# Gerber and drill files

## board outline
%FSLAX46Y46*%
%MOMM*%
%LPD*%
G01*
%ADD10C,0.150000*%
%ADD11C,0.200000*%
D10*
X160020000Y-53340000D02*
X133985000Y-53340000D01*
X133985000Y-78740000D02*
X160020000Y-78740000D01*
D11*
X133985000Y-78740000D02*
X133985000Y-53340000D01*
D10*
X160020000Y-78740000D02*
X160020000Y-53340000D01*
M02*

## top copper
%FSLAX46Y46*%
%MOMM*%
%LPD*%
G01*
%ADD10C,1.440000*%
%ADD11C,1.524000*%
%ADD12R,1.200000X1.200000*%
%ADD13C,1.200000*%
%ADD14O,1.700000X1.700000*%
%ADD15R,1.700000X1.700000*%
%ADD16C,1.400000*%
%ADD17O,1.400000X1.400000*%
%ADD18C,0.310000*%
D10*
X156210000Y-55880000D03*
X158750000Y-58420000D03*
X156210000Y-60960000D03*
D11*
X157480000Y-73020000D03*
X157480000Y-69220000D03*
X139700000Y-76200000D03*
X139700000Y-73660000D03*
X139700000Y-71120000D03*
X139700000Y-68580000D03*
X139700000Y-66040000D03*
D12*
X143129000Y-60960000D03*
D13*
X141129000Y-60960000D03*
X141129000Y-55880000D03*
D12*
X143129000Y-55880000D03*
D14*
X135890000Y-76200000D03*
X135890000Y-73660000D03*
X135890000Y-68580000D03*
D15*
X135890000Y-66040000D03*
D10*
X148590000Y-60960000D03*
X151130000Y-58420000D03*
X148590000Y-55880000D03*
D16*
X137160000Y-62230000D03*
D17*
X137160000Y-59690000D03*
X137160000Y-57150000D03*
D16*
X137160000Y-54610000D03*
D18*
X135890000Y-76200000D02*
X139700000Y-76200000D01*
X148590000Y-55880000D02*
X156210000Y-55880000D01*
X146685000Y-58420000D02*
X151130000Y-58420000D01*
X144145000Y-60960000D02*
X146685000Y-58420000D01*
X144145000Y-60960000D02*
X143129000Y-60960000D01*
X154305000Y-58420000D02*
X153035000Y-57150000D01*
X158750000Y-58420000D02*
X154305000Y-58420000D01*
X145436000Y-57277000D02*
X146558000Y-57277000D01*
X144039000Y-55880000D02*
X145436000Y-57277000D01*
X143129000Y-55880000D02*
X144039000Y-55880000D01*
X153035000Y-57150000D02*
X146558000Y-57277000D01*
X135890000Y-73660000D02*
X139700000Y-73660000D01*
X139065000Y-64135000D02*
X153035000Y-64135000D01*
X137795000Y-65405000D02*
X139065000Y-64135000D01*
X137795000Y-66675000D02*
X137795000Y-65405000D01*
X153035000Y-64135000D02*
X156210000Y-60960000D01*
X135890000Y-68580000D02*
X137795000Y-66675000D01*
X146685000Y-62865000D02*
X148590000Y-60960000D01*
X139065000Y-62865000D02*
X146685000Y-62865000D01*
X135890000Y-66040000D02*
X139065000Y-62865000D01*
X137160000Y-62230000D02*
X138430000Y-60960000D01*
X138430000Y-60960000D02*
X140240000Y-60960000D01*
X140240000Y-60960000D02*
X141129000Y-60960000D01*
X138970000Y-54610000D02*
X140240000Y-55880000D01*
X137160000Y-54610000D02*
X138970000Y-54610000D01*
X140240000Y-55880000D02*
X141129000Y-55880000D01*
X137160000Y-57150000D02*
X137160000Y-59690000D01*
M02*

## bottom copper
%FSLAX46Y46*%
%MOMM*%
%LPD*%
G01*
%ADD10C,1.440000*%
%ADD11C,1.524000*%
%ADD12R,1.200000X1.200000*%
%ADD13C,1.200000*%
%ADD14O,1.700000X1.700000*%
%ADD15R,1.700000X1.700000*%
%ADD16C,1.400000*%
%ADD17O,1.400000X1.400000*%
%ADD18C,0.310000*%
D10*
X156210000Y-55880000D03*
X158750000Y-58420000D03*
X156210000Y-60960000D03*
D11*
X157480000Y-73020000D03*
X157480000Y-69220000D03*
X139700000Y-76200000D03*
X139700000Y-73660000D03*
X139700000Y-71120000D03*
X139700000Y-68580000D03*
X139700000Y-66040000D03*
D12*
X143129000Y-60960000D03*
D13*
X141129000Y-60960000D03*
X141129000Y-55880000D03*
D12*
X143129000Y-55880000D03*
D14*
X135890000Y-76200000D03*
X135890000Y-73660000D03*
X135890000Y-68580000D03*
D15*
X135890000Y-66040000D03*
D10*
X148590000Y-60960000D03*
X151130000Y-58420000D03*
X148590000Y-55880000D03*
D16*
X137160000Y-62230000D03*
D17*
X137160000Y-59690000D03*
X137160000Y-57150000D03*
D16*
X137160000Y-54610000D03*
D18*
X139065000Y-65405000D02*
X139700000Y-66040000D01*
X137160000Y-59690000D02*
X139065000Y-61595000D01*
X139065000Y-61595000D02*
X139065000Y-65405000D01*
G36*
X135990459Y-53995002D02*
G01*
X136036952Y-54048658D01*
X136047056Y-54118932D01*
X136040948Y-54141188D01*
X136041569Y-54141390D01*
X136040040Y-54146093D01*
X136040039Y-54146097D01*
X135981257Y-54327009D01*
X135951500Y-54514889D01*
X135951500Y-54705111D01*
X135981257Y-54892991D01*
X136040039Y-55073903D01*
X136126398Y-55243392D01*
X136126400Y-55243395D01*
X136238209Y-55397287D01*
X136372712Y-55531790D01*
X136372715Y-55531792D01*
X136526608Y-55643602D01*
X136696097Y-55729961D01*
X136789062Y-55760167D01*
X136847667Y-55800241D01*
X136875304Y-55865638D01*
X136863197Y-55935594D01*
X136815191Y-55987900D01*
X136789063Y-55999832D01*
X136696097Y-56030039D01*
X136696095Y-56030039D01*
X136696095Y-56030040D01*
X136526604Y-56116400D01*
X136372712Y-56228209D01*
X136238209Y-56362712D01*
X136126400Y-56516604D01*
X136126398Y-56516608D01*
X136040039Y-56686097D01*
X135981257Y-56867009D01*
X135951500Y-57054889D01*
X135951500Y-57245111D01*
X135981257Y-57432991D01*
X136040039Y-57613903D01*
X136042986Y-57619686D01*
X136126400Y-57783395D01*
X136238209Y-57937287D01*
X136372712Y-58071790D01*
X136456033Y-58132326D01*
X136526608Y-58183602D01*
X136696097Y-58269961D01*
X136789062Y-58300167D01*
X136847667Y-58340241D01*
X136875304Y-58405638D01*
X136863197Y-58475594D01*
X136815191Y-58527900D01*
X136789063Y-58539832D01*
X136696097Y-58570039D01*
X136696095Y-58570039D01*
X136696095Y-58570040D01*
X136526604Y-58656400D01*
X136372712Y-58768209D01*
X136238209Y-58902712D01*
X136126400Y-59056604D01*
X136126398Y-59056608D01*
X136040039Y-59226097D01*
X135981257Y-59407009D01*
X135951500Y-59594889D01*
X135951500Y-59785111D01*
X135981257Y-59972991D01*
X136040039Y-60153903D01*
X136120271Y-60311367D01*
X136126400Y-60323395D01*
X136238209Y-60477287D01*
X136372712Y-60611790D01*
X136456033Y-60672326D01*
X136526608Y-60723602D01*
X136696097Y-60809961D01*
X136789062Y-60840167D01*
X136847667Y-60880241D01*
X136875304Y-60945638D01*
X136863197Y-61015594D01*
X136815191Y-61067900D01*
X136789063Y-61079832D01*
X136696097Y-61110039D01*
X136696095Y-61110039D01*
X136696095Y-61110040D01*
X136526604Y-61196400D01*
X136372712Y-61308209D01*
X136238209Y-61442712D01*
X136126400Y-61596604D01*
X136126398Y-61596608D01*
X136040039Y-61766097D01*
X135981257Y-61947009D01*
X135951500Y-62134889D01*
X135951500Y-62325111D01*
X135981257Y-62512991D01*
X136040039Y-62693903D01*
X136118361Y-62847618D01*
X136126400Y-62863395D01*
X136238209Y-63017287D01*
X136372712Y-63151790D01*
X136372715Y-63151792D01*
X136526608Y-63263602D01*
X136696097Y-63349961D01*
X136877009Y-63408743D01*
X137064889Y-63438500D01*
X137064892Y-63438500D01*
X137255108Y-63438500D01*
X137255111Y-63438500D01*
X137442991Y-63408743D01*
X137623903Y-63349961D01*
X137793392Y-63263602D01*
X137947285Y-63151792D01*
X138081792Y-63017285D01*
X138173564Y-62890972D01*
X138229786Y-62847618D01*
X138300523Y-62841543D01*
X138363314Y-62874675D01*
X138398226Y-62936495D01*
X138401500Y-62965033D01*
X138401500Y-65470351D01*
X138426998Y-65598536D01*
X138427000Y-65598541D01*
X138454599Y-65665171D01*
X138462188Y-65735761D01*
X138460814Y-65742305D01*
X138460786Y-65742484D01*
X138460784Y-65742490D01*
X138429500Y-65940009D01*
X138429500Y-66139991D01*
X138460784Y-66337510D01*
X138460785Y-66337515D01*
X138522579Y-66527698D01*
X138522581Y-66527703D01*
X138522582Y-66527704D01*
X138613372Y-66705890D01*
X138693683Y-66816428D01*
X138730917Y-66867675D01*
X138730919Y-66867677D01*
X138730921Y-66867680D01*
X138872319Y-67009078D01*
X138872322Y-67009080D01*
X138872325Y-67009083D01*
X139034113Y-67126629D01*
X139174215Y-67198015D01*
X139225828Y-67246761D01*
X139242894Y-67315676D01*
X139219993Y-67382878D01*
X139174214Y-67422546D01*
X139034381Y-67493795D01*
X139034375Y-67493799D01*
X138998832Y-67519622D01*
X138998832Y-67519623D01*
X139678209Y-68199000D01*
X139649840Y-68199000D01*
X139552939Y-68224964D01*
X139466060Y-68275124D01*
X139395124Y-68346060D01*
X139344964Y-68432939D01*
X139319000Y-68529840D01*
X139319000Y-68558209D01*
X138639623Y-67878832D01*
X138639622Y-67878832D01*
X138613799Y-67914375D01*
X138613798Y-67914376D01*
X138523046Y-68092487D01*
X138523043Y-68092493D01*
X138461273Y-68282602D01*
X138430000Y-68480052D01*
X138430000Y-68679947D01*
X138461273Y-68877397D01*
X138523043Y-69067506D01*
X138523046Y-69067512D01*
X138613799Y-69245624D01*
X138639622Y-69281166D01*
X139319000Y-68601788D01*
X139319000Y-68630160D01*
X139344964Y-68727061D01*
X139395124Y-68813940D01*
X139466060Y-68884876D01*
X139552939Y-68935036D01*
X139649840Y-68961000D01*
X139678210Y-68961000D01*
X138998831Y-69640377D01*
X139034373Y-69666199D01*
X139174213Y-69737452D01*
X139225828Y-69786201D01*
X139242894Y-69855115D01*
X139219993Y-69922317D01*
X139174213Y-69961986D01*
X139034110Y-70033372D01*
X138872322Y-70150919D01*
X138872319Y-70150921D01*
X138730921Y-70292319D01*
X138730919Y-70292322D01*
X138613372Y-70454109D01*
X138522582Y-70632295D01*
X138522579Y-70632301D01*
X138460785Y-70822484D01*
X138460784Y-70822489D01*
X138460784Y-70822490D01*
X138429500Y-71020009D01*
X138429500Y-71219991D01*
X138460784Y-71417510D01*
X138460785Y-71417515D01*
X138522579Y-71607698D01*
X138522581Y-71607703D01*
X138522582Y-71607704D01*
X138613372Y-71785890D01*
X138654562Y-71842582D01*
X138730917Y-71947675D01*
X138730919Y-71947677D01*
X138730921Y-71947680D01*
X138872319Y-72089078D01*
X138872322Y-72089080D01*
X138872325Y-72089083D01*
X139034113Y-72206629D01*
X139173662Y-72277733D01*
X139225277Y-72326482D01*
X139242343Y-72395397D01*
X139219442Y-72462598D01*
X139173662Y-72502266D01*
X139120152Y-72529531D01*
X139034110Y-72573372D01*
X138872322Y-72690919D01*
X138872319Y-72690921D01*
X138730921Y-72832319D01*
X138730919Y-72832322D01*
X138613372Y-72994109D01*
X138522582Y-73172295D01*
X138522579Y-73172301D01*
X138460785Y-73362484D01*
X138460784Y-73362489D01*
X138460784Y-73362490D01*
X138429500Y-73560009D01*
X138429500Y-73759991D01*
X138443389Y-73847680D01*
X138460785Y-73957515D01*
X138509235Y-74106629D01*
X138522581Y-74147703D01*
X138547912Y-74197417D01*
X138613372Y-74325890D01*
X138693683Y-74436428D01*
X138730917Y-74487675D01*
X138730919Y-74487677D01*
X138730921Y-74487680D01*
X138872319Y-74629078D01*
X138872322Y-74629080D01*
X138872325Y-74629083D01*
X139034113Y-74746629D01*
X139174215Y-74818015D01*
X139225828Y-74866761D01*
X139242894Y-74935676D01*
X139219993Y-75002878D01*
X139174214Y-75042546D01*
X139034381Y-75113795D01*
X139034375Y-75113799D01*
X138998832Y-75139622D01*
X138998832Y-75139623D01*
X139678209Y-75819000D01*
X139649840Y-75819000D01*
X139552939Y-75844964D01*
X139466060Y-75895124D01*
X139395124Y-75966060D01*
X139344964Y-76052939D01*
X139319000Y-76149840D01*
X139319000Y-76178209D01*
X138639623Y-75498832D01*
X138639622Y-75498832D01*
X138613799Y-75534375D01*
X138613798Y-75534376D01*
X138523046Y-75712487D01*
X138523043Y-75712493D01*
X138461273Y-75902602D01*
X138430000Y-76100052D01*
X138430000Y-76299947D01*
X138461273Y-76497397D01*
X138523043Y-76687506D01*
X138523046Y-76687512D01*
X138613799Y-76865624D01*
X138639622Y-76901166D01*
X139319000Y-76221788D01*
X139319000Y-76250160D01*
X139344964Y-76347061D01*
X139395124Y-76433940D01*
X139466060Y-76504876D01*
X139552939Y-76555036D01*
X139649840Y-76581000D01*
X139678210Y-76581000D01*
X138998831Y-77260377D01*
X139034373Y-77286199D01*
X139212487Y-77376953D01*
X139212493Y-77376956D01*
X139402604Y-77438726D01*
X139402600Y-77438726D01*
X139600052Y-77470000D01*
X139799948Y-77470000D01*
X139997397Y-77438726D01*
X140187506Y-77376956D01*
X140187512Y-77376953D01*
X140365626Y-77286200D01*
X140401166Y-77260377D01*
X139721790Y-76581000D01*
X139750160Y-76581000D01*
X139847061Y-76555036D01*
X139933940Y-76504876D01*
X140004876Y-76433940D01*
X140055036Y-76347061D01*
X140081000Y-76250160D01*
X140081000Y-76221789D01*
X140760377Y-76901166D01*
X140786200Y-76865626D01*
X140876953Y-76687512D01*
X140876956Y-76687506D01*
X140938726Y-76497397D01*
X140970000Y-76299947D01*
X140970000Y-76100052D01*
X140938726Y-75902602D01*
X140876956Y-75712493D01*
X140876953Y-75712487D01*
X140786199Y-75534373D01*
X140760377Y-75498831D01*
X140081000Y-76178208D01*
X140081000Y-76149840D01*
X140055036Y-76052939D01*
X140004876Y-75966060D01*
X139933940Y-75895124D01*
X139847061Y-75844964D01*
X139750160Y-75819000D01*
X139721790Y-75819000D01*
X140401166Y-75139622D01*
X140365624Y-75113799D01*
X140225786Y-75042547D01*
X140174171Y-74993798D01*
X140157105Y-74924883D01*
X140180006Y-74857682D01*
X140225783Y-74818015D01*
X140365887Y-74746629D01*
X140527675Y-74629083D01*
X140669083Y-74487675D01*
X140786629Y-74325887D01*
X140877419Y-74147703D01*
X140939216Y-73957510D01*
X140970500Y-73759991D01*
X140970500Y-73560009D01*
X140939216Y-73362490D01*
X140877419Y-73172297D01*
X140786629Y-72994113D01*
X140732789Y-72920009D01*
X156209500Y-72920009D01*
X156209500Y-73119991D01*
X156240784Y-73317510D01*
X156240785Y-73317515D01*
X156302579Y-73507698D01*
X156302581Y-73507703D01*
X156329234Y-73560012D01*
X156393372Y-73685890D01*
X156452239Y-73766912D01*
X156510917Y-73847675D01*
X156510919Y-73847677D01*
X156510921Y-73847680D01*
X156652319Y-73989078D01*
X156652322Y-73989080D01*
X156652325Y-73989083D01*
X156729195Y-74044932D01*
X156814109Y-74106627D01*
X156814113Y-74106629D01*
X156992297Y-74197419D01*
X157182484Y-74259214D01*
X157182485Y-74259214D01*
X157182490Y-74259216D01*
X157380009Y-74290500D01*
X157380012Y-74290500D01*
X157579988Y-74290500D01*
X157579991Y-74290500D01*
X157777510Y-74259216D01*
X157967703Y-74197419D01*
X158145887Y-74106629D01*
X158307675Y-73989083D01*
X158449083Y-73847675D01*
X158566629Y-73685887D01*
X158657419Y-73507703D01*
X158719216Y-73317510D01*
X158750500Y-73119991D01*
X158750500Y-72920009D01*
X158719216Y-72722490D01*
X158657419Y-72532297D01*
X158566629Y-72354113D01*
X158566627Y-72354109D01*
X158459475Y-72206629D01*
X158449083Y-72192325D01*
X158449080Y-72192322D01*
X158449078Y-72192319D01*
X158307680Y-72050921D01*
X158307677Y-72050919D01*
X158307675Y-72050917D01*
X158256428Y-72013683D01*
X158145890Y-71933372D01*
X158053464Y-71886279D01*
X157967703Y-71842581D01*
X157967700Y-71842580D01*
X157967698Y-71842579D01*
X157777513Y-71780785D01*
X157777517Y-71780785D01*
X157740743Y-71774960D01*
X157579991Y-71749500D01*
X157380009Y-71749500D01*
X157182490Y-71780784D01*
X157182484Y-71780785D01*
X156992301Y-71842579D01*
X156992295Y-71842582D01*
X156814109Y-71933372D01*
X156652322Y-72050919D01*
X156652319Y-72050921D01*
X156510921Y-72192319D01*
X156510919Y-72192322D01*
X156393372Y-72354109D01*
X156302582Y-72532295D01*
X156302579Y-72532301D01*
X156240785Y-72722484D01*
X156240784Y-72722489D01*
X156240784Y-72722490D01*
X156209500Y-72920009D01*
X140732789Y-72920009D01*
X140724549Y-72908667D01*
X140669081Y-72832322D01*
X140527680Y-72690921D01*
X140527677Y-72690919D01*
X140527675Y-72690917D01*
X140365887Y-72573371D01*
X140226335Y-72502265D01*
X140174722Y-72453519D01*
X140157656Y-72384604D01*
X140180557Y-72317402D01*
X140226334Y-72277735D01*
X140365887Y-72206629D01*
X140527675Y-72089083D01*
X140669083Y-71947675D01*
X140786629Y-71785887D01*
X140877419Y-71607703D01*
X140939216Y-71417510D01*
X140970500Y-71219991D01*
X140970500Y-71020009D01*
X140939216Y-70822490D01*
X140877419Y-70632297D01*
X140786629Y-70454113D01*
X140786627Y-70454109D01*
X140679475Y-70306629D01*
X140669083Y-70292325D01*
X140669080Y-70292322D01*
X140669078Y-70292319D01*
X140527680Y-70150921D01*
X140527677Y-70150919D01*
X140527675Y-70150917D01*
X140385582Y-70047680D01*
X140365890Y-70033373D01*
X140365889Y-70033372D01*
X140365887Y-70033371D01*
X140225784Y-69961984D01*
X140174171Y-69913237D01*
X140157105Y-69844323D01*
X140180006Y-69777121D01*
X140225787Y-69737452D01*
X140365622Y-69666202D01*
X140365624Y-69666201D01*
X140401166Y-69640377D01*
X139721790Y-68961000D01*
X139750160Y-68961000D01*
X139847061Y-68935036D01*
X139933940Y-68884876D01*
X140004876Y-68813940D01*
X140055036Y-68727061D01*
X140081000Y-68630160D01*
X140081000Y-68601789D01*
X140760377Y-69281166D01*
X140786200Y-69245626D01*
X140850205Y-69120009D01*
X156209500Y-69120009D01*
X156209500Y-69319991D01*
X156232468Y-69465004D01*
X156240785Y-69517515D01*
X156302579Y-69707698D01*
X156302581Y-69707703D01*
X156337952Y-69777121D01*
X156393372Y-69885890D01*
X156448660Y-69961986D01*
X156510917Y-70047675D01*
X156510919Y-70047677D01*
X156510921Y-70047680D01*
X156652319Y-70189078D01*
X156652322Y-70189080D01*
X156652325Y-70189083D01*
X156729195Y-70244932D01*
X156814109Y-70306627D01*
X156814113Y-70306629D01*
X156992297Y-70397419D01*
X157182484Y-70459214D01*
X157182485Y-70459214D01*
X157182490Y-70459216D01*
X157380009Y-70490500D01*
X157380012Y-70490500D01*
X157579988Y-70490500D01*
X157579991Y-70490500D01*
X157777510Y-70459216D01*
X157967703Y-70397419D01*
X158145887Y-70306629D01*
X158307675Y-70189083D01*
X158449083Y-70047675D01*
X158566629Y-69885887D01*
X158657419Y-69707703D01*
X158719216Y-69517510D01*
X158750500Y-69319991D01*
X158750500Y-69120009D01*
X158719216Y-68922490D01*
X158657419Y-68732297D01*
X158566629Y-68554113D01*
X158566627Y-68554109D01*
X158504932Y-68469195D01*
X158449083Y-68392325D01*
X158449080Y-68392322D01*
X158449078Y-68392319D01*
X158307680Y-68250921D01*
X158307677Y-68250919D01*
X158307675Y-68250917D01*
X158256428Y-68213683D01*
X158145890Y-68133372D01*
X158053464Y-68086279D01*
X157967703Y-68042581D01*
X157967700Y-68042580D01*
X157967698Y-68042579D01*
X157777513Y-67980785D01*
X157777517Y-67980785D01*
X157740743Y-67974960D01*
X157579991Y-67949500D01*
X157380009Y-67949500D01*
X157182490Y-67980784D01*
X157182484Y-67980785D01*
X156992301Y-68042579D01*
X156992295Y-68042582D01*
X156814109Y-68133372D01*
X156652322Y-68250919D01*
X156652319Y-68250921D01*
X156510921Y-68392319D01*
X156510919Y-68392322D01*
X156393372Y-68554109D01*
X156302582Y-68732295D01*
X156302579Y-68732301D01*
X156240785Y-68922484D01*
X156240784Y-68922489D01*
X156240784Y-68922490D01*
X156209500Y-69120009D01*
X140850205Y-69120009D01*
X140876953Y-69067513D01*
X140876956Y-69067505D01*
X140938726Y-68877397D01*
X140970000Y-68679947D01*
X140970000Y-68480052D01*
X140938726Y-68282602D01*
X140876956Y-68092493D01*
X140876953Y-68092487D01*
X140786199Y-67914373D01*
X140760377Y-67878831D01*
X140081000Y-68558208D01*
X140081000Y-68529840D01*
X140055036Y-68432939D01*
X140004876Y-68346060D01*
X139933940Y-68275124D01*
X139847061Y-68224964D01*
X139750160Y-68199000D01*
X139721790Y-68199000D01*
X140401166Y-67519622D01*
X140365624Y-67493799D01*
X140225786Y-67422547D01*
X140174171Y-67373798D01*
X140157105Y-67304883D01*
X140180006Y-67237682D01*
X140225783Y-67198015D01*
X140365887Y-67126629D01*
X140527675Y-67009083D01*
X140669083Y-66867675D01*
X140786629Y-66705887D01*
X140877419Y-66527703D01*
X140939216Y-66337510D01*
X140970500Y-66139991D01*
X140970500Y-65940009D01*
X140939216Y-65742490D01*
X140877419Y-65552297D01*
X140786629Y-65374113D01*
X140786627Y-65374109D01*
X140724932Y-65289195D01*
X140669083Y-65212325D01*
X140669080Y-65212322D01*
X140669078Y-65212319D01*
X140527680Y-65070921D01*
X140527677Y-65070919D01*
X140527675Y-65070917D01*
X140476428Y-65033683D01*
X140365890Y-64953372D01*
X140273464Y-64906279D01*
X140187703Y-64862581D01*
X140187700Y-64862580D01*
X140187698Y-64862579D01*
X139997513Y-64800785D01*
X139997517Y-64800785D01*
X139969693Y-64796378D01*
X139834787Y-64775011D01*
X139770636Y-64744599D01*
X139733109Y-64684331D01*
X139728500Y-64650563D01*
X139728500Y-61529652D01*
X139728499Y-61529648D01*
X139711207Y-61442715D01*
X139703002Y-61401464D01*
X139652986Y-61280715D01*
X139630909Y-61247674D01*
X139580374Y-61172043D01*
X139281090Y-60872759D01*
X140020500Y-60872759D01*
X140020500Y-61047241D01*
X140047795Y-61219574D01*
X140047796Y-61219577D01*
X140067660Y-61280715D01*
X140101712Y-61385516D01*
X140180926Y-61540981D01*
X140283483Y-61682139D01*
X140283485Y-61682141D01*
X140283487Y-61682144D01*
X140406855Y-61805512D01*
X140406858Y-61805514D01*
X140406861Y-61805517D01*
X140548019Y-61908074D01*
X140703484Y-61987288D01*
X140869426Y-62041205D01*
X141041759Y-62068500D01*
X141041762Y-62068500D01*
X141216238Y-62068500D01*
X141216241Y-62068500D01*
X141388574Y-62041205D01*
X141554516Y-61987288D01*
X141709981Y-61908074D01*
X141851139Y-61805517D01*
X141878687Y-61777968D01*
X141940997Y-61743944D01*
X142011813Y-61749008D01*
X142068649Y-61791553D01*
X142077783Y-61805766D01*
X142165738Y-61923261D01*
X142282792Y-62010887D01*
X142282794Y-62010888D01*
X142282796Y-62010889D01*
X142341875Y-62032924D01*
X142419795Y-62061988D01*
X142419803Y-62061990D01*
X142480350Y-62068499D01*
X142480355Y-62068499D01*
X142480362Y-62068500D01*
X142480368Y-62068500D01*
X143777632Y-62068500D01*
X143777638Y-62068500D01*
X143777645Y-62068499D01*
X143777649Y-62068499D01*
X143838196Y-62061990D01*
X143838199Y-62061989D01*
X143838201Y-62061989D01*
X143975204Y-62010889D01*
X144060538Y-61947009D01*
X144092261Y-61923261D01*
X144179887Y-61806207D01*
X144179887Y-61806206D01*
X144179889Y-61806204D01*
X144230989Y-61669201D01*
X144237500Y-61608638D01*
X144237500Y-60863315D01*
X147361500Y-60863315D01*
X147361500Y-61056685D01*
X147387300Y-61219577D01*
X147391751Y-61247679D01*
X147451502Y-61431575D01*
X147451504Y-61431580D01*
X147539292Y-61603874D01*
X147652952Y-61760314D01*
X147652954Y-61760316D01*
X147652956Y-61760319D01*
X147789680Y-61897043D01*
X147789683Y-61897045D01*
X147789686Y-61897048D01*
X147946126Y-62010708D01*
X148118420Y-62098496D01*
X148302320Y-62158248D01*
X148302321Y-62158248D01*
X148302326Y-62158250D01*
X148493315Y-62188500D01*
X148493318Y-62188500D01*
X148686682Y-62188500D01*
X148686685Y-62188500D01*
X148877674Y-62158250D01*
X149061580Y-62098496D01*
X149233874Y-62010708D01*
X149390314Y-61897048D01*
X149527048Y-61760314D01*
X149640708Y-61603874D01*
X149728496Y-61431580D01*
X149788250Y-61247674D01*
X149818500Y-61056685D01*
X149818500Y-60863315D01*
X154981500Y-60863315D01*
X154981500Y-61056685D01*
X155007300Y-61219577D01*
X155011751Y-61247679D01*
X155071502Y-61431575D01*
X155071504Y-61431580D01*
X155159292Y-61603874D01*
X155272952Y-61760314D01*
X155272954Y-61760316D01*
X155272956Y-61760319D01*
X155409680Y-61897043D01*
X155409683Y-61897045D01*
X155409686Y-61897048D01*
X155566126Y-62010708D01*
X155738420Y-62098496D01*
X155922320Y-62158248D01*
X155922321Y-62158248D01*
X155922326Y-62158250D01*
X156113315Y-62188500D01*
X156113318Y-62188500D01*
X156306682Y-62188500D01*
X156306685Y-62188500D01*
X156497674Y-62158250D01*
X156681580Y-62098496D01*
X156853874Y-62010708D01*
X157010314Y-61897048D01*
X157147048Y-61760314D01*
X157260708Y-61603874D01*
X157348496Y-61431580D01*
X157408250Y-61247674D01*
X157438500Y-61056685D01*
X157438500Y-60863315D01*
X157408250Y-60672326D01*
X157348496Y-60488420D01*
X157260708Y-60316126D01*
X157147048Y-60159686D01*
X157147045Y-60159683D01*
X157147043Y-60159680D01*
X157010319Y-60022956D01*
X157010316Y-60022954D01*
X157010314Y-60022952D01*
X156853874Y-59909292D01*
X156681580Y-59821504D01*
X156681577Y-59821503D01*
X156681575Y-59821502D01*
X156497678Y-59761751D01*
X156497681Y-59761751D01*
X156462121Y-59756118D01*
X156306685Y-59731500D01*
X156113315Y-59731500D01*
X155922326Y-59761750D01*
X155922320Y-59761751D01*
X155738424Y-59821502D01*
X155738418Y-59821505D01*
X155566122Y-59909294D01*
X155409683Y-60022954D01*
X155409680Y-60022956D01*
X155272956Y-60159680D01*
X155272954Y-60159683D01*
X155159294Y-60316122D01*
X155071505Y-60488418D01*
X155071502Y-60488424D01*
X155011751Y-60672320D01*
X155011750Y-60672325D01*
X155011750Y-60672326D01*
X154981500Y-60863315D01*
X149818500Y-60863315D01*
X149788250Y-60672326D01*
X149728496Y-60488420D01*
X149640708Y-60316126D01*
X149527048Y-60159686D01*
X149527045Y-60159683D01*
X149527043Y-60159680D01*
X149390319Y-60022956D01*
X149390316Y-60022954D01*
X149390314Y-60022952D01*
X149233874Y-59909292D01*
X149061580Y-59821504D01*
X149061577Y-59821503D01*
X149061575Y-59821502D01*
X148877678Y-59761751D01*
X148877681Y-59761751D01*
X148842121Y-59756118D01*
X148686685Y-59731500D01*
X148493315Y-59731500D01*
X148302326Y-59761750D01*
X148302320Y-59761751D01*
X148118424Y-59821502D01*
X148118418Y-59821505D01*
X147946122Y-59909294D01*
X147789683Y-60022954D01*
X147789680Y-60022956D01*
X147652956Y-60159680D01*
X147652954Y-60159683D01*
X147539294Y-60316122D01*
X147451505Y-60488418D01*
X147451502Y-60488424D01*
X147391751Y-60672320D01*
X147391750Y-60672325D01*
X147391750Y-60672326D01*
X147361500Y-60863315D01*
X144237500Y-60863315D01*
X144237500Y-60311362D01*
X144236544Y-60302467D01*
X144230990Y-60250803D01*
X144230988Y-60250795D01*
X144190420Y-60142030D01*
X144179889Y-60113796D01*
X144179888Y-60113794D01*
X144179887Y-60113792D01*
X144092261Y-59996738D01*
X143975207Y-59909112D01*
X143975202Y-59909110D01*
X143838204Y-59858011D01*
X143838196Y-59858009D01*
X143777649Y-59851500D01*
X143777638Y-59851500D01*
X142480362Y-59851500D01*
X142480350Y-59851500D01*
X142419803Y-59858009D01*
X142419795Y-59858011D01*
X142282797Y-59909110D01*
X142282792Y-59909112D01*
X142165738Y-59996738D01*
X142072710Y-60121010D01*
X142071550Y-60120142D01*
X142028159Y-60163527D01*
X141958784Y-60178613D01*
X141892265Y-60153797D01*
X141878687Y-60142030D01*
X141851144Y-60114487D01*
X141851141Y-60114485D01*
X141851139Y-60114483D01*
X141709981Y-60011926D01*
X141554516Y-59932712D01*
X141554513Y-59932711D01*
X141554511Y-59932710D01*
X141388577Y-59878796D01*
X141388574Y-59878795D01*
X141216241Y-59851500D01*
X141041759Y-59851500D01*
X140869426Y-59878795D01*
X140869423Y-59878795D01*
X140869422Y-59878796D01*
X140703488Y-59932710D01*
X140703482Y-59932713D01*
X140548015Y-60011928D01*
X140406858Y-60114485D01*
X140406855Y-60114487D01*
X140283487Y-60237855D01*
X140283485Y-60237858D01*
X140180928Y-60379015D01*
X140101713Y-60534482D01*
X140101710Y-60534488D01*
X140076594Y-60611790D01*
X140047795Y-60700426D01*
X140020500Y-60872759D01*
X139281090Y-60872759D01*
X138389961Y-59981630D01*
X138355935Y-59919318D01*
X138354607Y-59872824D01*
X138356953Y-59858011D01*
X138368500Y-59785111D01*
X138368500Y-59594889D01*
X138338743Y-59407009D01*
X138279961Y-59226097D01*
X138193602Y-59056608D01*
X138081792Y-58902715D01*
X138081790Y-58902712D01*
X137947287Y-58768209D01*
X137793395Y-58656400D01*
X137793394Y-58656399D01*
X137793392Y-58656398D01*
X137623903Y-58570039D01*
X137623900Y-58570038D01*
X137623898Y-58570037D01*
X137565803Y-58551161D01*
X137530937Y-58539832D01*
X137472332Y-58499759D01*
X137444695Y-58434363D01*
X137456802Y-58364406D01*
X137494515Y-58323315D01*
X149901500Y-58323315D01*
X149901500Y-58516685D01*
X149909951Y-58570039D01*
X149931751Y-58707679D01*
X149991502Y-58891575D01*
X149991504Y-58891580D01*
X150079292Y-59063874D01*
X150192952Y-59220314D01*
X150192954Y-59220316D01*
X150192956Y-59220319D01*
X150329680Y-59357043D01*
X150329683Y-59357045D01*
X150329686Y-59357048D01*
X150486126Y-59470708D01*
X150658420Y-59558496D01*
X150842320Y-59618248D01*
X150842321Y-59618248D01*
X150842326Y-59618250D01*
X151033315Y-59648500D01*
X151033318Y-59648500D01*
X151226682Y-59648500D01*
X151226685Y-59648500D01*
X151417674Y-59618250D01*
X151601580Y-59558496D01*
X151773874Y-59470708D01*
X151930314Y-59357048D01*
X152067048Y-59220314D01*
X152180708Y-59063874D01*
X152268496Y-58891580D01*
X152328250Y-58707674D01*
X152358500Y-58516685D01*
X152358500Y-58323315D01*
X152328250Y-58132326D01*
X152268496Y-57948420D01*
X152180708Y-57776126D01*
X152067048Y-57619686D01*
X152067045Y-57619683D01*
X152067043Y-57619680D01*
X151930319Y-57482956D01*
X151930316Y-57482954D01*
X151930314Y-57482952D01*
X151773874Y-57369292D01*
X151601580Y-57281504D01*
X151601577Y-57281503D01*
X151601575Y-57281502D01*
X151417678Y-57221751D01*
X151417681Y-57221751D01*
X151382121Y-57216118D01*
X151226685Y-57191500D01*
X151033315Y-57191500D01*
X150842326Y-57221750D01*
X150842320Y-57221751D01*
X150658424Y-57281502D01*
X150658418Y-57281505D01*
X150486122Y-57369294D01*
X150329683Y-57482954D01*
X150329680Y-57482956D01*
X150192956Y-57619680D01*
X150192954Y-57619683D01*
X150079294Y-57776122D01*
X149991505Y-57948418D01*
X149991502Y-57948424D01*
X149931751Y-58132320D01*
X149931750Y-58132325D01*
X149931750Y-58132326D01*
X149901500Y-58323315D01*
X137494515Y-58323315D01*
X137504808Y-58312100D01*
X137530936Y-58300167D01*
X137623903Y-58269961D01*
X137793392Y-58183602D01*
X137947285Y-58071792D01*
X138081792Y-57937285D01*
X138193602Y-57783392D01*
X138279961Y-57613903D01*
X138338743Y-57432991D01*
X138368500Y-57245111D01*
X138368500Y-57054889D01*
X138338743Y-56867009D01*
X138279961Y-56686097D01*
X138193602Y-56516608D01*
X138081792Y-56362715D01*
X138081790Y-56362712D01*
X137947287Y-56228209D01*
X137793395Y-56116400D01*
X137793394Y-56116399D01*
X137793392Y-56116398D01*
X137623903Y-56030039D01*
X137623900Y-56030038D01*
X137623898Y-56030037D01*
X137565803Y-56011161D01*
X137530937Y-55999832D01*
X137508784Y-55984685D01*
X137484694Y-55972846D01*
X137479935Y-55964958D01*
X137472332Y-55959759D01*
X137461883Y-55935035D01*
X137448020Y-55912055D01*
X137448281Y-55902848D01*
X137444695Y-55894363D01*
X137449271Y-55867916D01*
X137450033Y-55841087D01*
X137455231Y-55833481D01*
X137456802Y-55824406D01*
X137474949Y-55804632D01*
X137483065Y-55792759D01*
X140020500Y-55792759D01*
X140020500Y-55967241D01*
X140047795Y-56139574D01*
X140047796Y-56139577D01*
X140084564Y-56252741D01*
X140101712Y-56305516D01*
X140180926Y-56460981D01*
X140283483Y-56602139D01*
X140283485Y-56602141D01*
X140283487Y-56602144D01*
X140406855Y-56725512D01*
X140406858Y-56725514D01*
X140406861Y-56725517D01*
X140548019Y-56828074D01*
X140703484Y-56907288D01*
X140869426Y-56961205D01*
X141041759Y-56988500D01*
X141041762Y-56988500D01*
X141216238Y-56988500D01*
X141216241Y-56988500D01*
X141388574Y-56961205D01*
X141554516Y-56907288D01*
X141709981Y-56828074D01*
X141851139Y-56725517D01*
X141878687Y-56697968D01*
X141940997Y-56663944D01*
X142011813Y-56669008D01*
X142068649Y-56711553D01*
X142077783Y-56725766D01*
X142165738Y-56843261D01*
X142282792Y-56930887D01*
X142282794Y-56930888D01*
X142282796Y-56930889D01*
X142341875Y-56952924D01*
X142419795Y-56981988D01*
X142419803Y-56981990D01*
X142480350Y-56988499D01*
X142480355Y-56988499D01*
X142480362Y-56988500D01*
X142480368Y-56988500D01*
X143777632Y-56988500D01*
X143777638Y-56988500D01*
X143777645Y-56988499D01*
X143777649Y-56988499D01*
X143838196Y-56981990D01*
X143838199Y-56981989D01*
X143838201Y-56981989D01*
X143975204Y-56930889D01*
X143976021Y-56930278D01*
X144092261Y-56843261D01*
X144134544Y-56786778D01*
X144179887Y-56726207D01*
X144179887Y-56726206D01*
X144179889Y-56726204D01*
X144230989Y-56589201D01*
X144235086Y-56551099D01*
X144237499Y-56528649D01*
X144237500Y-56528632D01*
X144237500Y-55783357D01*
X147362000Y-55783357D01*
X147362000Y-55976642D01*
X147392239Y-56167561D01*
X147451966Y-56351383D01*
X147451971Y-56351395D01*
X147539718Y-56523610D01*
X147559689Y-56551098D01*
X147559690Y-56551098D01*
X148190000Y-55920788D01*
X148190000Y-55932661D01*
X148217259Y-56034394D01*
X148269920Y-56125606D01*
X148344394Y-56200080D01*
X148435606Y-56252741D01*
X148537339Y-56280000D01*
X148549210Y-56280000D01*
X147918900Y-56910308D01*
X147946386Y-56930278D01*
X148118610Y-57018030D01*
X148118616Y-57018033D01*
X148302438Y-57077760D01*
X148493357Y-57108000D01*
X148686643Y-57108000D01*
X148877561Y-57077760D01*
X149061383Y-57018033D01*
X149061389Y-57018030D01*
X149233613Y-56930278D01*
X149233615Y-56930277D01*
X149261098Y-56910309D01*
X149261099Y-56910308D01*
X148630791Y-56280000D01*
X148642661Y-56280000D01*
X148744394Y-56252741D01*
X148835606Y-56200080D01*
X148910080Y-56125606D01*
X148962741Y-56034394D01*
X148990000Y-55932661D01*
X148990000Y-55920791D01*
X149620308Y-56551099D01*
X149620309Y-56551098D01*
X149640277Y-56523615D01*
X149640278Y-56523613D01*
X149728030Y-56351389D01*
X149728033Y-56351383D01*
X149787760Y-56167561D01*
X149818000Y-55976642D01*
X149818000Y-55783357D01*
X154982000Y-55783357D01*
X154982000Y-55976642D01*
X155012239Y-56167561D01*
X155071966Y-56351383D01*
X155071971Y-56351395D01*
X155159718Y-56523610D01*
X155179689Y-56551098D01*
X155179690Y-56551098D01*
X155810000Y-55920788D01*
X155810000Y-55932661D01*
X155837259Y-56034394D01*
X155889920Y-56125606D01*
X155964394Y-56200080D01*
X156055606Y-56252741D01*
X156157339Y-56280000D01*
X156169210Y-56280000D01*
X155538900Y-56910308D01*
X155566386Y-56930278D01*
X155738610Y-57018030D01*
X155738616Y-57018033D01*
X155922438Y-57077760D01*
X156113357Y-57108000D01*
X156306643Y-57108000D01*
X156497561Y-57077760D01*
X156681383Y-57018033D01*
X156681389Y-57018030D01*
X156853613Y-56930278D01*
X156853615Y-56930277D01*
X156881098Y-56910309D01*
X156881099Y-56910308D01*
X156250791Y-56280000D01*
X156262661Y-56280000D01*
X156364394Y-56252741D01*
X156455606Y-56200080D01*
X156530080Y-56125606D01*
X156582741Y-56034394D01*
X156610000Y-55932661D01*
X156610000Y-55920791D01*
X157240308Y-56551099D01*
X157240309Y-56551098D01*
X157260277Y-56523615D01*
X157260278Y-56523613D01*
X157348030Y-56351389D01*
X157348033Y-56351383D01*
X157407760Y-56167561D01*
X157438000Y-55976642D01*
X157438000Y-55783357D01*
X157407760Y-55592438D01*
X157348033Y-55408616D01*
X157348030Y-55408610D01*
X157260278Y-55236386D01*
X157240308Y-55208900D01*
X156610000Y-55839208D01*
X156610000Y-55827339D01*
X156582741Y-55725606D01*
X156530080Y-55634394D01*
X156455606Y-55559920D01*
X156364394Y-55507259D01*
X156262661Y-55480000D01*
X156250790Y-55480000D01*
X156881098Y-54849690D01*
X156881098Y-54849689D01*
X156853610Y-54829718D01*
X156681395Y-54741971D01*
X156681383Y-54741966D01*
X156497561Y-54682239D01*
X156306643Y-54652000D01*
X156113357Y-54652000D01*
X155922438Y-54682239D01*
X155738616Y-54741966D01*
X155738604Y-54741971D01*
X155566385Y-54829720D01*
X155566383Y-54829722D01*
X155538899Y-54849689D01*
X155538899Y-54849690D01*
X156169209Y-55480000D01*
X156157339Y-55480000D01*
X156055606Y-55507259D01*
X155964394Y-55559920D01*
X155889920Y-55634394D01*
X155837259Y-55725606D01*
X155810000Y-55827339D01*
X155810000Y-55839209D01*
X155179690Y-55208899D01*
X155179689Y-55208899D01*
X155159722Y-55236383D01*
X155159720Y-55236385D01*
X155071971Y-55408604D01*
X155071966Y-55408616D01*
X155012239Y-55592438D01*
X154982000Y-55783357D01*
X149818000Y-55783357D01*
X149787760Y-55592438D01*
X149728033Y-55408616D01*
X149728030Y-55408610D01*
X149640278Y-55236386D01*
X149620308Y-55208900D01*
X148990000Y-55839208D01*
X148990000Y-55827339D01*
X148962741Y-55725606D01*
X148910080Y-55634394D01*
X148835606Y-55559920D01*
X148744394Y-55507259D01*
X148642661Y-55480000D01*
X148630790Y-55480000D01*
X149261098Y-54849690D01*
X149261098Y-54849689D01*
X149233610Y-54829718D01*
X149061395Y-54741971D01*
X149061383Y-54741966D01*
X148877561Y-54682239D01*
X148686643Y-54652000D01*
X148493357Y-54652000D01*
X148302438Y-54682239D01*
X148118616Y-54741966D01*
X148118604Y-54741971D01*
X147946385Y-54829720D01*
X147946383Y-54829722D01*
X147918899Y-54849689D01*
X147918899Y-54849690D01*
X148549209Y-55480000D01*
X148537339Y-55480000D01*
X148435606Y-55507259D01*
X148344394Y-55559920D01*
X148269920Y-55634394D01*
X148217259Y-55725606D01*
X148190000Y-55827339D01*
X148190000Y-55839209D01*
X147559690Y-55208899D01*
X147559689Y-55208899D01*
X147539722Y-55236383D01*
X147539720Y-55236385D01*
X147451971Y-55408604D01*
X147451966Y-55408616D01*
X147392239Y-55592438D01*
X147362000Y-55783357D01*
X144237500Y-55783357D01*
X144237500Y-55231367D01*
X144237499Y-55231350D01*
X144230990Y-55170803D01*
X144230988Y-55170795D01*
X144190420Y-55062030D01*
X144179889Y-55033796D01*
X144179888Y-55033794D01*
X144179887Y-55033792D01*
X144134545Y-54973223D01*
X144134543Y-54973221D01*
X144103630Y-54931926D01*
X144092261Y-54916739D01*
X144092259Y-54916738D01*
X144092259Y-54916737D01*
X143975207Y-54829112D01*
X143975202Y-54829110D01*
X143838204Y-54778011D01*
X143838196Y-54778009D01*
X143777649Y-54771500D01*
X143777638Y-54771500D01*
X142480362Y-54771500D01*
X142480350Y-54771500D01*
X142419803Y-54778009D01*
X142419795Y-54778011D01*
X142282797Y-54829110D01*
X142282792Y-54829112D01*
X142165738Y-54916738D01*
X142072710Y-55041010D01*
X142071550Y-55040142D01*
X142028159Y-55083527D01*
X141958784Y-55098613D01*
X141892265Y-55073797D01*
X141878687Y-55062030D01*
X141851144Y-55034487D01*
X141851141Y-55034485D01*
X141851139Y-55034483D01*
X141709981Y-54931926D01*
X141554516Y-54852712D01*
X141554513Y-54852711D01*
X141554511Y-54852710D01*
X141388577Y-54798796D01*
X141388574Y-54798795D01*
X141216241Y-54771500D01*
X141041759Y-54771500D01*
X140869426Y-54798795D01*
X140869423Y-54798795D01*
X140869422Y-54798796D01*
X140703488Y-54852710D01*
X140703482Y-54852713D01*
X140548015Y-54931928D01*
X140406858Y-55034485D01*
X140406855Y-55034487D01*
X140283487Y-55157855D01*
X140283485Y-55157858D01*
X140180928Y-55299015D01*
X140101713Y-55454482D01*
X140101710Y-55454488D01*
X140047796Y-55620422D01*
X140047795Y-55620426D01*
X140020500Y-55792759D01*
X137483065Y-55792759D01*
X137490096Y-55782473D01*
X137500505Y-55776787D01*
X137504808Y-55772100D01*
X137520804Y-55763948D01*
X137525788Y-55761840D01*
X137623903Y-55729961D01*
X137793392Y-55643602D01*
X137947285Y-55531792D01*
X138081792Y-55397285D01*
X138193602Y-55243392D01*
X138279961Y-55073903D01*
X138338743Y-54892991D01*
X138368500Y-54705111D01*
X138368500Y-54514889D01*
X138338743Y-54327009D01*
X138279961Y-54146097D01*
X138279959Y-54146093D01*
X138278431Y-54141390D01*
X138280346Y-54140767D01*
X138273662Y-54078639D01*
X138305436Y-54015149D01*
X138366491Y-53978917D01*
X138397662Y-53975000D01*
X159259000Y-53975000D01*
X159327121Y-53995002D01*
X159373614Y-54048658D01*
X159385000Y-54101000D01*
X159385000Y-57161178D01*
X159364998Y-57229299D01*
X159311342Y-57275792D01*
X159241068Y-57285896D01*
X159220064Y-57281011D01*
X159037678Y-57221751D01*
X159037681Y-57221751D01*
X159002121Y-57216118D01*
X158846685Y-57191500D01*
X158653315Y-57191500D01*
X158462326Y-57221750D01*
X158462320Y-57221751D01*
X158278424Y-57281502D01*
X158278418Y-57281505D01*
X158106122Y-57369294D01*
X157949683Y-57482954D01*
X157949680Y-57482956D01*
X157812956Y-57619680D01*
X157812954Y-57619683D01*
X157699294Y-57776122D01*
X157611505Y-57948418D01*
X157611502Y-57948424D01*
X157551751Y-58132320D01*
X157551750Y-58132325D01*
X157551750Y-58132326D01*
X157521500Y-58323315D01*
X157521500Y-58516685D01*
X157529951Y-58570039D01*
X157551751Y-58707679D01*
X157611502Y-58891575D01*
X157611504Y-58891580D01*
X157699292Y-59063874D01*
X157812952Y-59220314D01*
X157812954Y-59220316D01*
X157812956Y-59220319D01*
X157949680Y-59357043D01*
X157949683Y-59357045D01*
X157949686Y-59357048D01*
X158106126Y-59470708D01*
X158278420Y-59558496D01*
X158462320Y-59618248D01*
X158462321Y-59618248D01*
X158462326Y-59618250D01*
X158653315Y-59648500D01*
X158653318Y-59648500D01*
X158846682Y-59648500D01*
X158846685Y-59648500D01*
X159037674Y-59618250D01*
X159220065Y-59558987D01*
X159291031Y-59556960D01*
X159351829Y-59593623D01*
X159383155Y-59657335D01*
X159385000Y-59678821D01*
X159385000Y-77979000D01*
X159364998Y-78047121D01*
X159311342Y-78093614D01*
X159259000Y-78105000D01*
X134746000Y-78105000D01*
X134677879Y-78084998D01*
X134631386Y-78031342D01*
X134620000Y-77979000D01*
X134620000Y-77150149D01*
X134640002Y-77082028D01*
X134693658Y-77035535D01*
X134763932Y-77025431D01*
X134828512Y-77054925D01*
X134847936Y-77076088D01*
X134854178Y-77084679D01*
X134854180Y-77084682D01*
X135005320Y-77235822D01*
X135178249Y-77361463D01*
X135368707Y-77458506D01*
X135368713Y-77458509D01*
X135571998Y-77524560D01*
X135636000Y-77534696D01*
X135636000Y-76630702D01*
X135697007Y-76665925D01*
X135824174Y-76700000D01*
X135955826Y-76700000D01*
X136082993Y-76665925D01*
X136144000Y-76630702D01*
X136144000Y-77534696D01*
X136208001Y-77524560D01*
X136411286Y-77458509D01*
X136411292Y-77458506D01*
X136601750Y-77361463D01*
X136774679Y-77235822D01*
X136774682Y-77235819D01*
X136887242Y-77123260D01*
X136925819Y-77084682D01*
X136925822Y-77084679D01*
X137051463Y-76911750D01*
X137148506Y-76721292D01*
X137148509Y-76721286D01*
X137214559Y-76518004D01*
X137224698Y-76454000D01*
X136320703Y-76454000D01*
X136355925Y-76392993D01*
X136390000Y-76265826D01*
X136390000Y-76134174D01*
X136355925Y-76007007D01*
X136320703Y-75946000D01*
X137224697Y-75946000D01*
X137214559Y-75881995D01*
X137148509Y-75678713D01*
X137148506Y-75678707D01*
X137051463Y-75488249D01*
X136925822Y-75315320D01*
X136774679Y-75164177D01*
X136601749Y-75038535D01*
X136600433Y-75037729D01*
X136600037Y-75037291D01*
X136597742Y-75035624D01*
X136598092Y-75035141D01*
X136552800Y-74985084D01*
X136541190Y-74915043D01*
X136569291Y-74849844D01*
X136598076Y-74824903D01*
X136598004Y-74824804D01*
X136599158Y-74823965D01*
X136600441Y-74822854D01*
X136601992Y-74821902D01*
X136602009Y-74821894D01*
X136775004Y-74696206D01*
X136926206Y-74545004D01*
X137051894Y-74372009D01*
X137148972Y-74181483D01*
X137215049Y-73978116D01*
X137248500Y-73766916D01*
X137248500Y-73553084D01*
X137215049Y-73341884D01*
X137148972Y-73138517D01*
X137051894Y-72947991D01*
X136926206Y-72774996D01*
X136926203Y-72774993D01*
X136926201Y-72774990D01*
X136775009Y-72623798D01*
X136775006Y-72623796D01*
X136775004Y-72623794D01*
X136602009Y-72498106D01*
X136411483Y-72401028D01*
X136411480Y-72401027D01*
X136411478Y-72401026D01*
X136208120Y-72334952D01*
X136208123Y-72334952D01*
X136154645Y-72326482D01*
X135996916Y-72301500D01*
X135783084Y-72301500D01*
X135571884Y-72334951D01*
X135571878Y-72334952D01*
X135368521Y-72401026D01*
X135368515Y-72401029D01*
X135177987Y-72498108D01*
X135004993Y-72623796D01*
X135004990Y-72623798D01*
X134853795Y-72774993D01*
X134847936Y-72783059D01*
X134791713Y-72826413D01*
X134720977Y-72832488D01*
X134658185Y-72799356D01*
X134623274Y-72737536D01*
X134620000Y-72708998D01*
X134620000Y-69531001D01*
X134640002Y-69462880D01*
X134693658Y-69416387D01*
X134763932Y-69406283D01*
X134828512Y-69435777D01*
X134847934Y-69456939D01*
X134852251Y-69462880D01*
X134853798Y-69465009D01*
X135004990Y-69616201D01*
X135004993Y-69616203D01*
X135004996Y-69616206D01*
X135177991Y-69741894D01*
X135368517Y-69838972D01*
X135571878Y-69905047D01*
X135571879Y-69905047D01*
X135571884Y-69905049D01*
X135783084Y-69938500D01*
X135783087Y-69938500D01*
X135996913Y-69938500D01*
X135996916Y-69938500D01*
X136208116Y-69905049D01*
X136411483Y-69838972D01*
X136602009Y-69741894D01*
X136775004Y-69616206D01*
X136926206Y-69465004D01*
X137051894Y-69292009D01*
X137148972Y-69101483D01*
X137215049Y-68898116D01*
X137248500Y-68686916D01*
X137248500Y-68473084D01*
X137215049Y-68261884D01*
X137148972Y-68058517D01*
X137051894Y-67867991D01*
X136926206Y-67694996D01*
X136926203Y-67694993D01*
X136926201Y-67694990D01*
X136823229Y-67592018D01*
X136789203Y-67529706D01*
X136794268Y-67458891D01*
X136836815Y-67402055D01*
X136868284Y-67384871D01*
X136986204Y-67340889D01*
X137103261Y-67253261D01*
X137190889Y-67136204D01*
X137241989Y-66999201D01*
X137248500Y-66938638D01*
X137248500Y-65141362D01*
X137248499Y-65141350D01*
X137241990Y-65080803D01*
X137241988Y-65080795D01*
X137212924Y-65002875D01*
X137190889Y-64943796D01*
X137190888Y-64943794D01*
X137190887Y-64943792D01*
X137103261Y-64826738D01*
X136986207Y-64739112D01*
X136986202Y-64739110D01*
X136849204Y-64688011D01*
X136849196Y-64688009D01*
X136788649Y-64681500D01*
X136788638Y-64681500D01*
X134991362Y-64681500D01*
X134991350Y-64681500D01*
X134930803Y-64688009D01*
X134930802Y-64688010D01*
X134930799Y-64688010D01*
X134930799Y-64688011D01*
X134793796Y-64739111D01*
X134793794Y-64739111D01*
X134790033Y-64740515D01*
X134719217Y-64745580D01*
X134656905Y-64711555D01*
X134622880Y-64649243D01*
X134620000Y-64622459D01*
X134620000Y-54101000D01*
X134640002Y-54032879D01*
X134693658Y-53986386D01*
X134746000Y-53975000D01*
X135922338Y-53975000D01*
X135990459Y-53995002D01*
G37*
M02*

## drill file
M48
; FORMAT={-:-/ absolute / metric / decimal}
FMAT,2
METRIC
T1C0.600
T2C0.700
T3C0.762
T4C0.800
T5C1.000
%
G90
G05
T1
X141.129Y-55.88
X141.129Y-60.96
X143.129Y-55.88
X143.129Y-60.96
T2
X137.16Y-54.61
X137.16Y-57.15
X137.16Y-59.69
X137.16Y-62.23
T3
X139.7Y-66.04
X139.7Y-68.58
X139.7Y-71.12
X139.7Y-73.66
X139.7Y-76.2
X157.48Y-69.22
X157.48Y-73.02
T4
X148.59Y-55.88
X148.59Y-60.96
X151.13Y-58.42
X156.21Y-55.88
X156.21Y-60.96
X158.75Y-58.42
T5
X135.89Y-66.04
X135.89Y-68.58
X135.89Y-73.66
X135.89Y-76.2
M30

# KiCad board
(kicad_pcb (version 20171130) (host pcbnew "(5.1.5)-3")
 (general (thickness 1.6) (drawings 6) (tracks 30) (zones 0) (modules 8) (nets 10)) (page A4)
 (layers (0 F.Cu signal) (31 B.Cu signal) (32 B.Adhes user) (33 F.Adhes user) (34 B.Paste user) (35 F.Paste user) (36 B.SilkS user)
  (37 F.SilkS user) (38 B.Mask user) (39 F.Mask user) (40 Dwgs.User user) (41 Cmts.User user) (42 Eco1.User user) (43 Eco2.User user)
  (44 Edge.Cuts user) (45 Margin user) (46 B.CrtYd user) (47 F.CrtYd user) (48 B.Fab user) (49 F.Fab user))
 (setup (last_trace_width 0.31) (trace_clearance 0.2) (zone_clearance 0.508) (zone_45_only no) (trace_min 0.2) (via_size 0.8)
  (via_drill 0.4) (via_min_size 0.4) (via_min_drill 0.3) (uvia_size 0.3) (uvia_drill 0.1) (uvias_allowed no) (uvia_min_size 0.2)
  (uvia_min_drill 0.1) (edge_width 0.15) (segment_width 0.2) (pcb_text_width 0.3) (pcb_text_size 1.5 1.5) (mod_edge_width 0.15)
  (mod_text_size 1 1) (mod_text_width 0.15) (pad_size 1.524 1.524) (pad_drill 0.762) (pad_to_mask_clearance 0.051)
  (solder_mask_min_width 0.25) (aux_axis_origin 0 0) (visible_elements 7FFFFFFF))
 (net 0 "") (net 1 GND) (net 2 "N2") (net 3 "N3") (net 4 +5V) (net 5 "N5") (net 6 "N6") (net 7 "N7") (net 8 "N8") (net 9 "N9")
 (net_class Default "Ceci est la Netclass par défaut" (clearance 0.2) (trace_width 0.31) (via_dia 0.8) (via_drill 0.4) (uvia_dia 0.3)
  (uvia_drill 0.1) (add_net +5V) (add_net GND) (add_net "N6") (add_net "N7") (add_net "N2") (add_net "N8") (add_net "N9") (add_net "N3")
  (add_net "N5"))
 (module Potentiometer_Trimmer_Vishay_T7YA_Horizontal (layer F.Cu) (at 156.21 60.96)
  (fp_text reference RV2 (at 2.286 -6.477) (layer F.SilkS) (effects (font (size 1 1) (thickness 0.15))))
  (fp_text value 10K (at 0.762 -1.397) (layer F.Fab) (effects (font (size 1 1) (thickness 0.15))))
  (pad 3 thru_hole circle (at 0 -5.08) (size 1.44 1.44) (drill 0.8) (layers *.Cu *.Mask) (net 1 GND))
  (pad 2 thru_hole circle (at 2.54 -2.54) (size 1.44 1.44) (drill 0.8) (layers *.Cu *.Mask) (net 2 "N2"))
  (pad 1 thru_hole circle (at 0 0) (size 1.44 1.44) (drill 0.8) (layers *.Cu *.Mask) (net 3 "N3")))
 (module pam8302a (layer F.Cu) (at 139.7 71.12)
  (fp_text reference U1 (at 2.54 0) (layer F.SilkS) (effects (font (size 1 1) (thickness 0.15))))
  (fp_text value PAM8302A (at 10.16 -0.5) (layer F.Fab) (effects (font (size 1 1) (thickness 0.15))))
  (pad 7 thru_hole circle (at 17.78 1.9) (size 1.524 1.524) (drill 0.762) (layers *.Cu *.Mask))
  (pad 6 thru_hole circle (at 17.78 -1.9) (size 1.524 1.524) (drill 0.762) (layers *.Cu *.Mask))
  (pad 5 thru_hole circle (at 0 5.08) (size 1.524 1.524) (drill 0.762) (layers *.Cu *.Mask) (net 1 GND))
  (pad 4 thru_hole circle (at 0 2.54) (size 1.524 1.524) (drill 0.762) (layers *.Cu *.Mask) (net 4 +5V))
  (pad 3 thru_hole circle (at 0 0) (size 1.524 1.524) (drill 0.762) (layers *.Cu *.Mask))
  (pad 2 thru_hole circle (at 0 -2.54) (size 1.524 1.524) (drill 0.762) (layers *.Cu *.Mask) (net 1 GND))
  (pad 1 thru_hole circle (at 0 -5.08) (size 1.524 1.524) (drill 0.762) (layers *.Cu *.Mask) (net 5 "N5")))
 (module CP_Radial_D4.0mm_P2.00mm (layer F.Cu) (at 143.129 60.96 180)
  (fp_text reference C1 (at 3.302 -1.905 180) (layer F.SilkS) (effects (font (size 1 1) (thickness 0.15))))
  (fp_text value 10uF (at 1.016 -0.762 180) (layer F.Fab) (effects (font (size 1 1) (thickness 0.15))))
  (pad 1 thru_hole rect (at 0 0 180) (size 1.2 1.2) (drill 0.6) (layers *.Cu *.Mask) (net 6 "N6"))
  (pad 2 thru_hole circle (at 2 0 180) (size 1.2 1.2) (drill 0.6) (layers *.Cu *.Mask) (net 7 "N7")))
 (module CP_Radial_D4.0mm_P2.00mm (layer F.Cu) (at 143.129 55.88 180)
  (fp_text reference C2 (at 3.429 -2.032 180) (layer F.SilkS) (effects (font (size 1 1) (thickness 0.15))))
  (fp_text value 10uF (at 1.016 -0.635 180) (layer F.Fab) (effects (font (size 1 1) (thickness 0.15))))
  (pad 2 thru_hole circle (at 2 0 180) (size 1.2 1.2) (drill 0.6) (layers *.Cu *.Mask) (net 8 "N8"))
  (pad 1 thru_hole rect (at 0 0 180) (size 1.2 1.2) (drill 0.6) (layers *.Cu *.Mask) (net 2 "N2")))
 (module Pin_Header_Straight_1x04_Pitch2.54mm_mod (layer F.Cu) (at 135.89 66.04)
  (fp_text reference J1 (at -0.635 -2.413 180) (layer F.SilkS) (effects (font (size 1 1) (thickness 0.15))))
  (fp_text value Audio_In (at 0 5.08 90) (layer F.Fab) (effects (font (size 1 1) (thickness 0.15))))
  (pad 4 thru_hole oval (at 0 10.16) (size 1.7 1.7) (drill 1) (layers *.Cu *.Mask) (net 1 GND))
  (pad 3 thru_hole oval (at 0 7.62) (size 1.7 1.7) (drill 1) (layers *.Cu *.Mask) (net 4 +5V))
  (pad 2 thru_hole oval (at 0 2.54) (size 1.7 1.7) (drill 1) (layers *.Cu *.Mask) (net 3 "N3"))
  (pad 1 thru_hole rect (at 0 0) (size 1.7 1.7) (drill 1) (layers *.Cu *.Mask) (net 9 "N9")))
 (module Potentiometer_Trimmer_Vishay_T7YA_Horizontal (layer F.Cu) (at 148.59 60.96)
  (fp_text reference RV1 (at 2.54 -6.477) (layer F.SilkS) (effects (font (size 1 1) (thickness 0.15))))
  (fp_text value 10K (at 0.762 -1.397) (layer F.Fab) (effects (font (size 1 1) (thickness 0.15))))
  (pad 1 thru_hole circle (at 0 0) (size 1.44 1.44) (drill 0.8) (layers *.Cu *.Mask) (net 9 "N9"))
  (pad 2 thru_hole circle (at 2.54 -2.54) (size 1.44 1.44) (drill 0.8) (layers *.Cu *.Mask) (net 6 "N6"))
  (pad 3 thru_hole circle (at 0 -5.08) (size 1.44 1.44) (drill 0.8) (layers *.Cu *.Mask) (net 1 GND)))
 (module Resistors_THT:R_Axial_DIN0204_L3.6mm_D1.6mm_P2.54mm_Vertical (layer F.Cu) (at 137.16 62.23 90)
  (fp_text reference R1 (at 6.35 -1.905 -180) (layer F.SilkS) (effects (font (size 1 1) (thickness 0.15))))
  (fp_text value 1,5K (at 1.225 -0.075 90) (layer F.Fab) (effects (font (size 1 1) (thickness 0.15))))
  (pad 1 thru_hole circle (at 0 0 90) (size 1.4 1.4) (drill 0.7) (layers *.Cu *.Mask) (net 7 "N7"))
  (pad 2 thru_hole oval (at 2.54 0 90) (size 1.4 1.4) (drill 0.7) (layers *.Cu *.Mask) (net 5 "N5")))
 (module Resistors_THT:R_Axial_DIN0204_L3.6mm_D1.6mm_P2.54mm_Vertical (layer F.Cu) (at 137.16 54.61 270)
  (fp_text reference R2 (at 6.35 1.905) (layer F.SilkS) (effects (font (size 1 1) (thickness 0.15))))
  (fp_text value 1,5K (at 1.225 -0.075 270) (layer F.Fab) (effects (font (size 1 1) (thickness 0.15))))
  (pad 2 thru_hole oval (at 2.54 0 270) (size 1.4 1.4) (drill 0.7) (layers *.Cu *.Mask) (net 5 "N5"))
  (pad 1 thru_hole circle (at 0 0 270) (size 1.4 1.4) (drill 0.7) (layers *.Cu *.Mask) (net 8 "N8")))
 (gr_line (start 160.02 53.34) (end 133.985 53.34) (layer Edge.Cuts) (width 0.15))
 (gr_line (start 133.985 78.74) (end 160.02 78.74) (layer Edge.Cuts) (width 0.15))
 (gr_line (start 133.985 78.74) (end 133.985 53.34) (layer Edge.Cuts) (width 0.2))
 (gr_line (start 160.02 78.74) (end 160.02 53.34) (layer Edge.Cuts) (width 0.15))
 (segment (start 135.89 76.2) (end 139.7 76.2) (width 0.31) (layer F.Cu) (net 1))
 (segment (start 148.59 55.88) (end 156.21 55.88) (width 0.31) (layer F.Cu) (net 1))
 (segment (start 146.685 58.42) (end 151.13 58.42) (width 0.31) (layer F.Cu) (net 6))
 (segment (start 144.145 60.96) (end 146.685 58.42) (width 0.31) (layer F.Cu) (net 6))
 (segment (start 144.145 60.96) (end 143.129 60.96) (width 0.31) (layer F.Cu) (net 6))
 (segment (start 154.305 58.42) (end 153.035 57.15) (width 0.31) (layer F.Cu) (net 2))
 (segment (start 158.75 58.42) (end 154.305 58.42) (width 0.31) (layer F.Cu) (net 2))
 (segment (start 145.436 57.277) (end 146.558 57.277) (width 0.31) (layer F.Cu) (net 2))
 (segment (start 144.039 55.88) (end 145.436 57.277) (width 0.31) (layer F.Cu) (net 2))
 (segment (start 143.129 55.88) (end 144.039 55.88) (width 0.31) (layer F.Cu) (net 2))
 (segment (start 153.035 57.15) (end 146.558 57.277) (width 0.31) (layer F.Cu) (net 2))
 (segment (start 135.89 73.66) (end 139.7 73.66) (width 0.31) (layer F.Cu) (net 4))
 (segment (start 139.065 64.135) (end 153.035 64.135) (width 0.31) (layer F.Cu) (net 3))
 (segment (start 137.795 65.405) (end 139.065 64.135) (width 0.31) (layer F.Cu) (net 3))
 (segment (start 137.795 66.675) (end 137.795 65.405) (width 0.31) (layer F.Cu) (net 3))
 (segment (start 153.035 64.135) (end 156.21 60.96) (width 0.31) (layer F.Cu) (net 3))
 (segment (start 135.89 68.58) (end 137.795 66.675) (width 0.31) (layer F.Cu) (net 3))
 (segment (start 146.685 62.865) (end 148.59 60.96) (width 0.31) (layer F.Cu) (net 9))
 (segment (start 139.065 62.865) (end 146.685 62.865) (width 0.31) (layer F.Cu) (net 9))
 (segment (start 135.89 66.04) (end 139.065 62.865) (width 0.31) (layer F.Cu) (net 9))
 (segment (start 137.16 62.23) (end 138.43 60.96) (width 0.31) (layer F.Cu) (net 7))
 (segment (start 138.43 60.96) (end 140.24 60.96) (width 0.31) (layer F.Cu) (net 7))
 (segment (start 140.24 60.96) (end 141.129 60.96) (width 0.31) (layer F.Cu) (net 7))
 (segment (start 138.97 54.61) (end 140.24 55.88) (width 0.31) (layer F.Cu) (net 8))
 (segment (start 137.16 54.61) (end 138.97 54.61) (width 0.31) (layer F.Cu) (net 8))
 (segment (start 140.24 55.88) (end 141.129 55.88) (width 0.31) (layer F.Cu) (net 8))
 (segment (start 137.16 57.15) (end 137.16 59.69) (width 0.31) (layer F.Cu) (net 5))
 (segment (start 139.065 65.405) (end 139.7 66.04) (width 0.31) (layer B.Cu) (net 5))
 (segment (start 137.16 59.69) (end 139.065 61.595) (width 0.31) (layer B.Cu) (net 5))
 (segment (start 139.065 61.595) (end 139.065 65.405) (width 0.31) (layer B.Cu) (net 5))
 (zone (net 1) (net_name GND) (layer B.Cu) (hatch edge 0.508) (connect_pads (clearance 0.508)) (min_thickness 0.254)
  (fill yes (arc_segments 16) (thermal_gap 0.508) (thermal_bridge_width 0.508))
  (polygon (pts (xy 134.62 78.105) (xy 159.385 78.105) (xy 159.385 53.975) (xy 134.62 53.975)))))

